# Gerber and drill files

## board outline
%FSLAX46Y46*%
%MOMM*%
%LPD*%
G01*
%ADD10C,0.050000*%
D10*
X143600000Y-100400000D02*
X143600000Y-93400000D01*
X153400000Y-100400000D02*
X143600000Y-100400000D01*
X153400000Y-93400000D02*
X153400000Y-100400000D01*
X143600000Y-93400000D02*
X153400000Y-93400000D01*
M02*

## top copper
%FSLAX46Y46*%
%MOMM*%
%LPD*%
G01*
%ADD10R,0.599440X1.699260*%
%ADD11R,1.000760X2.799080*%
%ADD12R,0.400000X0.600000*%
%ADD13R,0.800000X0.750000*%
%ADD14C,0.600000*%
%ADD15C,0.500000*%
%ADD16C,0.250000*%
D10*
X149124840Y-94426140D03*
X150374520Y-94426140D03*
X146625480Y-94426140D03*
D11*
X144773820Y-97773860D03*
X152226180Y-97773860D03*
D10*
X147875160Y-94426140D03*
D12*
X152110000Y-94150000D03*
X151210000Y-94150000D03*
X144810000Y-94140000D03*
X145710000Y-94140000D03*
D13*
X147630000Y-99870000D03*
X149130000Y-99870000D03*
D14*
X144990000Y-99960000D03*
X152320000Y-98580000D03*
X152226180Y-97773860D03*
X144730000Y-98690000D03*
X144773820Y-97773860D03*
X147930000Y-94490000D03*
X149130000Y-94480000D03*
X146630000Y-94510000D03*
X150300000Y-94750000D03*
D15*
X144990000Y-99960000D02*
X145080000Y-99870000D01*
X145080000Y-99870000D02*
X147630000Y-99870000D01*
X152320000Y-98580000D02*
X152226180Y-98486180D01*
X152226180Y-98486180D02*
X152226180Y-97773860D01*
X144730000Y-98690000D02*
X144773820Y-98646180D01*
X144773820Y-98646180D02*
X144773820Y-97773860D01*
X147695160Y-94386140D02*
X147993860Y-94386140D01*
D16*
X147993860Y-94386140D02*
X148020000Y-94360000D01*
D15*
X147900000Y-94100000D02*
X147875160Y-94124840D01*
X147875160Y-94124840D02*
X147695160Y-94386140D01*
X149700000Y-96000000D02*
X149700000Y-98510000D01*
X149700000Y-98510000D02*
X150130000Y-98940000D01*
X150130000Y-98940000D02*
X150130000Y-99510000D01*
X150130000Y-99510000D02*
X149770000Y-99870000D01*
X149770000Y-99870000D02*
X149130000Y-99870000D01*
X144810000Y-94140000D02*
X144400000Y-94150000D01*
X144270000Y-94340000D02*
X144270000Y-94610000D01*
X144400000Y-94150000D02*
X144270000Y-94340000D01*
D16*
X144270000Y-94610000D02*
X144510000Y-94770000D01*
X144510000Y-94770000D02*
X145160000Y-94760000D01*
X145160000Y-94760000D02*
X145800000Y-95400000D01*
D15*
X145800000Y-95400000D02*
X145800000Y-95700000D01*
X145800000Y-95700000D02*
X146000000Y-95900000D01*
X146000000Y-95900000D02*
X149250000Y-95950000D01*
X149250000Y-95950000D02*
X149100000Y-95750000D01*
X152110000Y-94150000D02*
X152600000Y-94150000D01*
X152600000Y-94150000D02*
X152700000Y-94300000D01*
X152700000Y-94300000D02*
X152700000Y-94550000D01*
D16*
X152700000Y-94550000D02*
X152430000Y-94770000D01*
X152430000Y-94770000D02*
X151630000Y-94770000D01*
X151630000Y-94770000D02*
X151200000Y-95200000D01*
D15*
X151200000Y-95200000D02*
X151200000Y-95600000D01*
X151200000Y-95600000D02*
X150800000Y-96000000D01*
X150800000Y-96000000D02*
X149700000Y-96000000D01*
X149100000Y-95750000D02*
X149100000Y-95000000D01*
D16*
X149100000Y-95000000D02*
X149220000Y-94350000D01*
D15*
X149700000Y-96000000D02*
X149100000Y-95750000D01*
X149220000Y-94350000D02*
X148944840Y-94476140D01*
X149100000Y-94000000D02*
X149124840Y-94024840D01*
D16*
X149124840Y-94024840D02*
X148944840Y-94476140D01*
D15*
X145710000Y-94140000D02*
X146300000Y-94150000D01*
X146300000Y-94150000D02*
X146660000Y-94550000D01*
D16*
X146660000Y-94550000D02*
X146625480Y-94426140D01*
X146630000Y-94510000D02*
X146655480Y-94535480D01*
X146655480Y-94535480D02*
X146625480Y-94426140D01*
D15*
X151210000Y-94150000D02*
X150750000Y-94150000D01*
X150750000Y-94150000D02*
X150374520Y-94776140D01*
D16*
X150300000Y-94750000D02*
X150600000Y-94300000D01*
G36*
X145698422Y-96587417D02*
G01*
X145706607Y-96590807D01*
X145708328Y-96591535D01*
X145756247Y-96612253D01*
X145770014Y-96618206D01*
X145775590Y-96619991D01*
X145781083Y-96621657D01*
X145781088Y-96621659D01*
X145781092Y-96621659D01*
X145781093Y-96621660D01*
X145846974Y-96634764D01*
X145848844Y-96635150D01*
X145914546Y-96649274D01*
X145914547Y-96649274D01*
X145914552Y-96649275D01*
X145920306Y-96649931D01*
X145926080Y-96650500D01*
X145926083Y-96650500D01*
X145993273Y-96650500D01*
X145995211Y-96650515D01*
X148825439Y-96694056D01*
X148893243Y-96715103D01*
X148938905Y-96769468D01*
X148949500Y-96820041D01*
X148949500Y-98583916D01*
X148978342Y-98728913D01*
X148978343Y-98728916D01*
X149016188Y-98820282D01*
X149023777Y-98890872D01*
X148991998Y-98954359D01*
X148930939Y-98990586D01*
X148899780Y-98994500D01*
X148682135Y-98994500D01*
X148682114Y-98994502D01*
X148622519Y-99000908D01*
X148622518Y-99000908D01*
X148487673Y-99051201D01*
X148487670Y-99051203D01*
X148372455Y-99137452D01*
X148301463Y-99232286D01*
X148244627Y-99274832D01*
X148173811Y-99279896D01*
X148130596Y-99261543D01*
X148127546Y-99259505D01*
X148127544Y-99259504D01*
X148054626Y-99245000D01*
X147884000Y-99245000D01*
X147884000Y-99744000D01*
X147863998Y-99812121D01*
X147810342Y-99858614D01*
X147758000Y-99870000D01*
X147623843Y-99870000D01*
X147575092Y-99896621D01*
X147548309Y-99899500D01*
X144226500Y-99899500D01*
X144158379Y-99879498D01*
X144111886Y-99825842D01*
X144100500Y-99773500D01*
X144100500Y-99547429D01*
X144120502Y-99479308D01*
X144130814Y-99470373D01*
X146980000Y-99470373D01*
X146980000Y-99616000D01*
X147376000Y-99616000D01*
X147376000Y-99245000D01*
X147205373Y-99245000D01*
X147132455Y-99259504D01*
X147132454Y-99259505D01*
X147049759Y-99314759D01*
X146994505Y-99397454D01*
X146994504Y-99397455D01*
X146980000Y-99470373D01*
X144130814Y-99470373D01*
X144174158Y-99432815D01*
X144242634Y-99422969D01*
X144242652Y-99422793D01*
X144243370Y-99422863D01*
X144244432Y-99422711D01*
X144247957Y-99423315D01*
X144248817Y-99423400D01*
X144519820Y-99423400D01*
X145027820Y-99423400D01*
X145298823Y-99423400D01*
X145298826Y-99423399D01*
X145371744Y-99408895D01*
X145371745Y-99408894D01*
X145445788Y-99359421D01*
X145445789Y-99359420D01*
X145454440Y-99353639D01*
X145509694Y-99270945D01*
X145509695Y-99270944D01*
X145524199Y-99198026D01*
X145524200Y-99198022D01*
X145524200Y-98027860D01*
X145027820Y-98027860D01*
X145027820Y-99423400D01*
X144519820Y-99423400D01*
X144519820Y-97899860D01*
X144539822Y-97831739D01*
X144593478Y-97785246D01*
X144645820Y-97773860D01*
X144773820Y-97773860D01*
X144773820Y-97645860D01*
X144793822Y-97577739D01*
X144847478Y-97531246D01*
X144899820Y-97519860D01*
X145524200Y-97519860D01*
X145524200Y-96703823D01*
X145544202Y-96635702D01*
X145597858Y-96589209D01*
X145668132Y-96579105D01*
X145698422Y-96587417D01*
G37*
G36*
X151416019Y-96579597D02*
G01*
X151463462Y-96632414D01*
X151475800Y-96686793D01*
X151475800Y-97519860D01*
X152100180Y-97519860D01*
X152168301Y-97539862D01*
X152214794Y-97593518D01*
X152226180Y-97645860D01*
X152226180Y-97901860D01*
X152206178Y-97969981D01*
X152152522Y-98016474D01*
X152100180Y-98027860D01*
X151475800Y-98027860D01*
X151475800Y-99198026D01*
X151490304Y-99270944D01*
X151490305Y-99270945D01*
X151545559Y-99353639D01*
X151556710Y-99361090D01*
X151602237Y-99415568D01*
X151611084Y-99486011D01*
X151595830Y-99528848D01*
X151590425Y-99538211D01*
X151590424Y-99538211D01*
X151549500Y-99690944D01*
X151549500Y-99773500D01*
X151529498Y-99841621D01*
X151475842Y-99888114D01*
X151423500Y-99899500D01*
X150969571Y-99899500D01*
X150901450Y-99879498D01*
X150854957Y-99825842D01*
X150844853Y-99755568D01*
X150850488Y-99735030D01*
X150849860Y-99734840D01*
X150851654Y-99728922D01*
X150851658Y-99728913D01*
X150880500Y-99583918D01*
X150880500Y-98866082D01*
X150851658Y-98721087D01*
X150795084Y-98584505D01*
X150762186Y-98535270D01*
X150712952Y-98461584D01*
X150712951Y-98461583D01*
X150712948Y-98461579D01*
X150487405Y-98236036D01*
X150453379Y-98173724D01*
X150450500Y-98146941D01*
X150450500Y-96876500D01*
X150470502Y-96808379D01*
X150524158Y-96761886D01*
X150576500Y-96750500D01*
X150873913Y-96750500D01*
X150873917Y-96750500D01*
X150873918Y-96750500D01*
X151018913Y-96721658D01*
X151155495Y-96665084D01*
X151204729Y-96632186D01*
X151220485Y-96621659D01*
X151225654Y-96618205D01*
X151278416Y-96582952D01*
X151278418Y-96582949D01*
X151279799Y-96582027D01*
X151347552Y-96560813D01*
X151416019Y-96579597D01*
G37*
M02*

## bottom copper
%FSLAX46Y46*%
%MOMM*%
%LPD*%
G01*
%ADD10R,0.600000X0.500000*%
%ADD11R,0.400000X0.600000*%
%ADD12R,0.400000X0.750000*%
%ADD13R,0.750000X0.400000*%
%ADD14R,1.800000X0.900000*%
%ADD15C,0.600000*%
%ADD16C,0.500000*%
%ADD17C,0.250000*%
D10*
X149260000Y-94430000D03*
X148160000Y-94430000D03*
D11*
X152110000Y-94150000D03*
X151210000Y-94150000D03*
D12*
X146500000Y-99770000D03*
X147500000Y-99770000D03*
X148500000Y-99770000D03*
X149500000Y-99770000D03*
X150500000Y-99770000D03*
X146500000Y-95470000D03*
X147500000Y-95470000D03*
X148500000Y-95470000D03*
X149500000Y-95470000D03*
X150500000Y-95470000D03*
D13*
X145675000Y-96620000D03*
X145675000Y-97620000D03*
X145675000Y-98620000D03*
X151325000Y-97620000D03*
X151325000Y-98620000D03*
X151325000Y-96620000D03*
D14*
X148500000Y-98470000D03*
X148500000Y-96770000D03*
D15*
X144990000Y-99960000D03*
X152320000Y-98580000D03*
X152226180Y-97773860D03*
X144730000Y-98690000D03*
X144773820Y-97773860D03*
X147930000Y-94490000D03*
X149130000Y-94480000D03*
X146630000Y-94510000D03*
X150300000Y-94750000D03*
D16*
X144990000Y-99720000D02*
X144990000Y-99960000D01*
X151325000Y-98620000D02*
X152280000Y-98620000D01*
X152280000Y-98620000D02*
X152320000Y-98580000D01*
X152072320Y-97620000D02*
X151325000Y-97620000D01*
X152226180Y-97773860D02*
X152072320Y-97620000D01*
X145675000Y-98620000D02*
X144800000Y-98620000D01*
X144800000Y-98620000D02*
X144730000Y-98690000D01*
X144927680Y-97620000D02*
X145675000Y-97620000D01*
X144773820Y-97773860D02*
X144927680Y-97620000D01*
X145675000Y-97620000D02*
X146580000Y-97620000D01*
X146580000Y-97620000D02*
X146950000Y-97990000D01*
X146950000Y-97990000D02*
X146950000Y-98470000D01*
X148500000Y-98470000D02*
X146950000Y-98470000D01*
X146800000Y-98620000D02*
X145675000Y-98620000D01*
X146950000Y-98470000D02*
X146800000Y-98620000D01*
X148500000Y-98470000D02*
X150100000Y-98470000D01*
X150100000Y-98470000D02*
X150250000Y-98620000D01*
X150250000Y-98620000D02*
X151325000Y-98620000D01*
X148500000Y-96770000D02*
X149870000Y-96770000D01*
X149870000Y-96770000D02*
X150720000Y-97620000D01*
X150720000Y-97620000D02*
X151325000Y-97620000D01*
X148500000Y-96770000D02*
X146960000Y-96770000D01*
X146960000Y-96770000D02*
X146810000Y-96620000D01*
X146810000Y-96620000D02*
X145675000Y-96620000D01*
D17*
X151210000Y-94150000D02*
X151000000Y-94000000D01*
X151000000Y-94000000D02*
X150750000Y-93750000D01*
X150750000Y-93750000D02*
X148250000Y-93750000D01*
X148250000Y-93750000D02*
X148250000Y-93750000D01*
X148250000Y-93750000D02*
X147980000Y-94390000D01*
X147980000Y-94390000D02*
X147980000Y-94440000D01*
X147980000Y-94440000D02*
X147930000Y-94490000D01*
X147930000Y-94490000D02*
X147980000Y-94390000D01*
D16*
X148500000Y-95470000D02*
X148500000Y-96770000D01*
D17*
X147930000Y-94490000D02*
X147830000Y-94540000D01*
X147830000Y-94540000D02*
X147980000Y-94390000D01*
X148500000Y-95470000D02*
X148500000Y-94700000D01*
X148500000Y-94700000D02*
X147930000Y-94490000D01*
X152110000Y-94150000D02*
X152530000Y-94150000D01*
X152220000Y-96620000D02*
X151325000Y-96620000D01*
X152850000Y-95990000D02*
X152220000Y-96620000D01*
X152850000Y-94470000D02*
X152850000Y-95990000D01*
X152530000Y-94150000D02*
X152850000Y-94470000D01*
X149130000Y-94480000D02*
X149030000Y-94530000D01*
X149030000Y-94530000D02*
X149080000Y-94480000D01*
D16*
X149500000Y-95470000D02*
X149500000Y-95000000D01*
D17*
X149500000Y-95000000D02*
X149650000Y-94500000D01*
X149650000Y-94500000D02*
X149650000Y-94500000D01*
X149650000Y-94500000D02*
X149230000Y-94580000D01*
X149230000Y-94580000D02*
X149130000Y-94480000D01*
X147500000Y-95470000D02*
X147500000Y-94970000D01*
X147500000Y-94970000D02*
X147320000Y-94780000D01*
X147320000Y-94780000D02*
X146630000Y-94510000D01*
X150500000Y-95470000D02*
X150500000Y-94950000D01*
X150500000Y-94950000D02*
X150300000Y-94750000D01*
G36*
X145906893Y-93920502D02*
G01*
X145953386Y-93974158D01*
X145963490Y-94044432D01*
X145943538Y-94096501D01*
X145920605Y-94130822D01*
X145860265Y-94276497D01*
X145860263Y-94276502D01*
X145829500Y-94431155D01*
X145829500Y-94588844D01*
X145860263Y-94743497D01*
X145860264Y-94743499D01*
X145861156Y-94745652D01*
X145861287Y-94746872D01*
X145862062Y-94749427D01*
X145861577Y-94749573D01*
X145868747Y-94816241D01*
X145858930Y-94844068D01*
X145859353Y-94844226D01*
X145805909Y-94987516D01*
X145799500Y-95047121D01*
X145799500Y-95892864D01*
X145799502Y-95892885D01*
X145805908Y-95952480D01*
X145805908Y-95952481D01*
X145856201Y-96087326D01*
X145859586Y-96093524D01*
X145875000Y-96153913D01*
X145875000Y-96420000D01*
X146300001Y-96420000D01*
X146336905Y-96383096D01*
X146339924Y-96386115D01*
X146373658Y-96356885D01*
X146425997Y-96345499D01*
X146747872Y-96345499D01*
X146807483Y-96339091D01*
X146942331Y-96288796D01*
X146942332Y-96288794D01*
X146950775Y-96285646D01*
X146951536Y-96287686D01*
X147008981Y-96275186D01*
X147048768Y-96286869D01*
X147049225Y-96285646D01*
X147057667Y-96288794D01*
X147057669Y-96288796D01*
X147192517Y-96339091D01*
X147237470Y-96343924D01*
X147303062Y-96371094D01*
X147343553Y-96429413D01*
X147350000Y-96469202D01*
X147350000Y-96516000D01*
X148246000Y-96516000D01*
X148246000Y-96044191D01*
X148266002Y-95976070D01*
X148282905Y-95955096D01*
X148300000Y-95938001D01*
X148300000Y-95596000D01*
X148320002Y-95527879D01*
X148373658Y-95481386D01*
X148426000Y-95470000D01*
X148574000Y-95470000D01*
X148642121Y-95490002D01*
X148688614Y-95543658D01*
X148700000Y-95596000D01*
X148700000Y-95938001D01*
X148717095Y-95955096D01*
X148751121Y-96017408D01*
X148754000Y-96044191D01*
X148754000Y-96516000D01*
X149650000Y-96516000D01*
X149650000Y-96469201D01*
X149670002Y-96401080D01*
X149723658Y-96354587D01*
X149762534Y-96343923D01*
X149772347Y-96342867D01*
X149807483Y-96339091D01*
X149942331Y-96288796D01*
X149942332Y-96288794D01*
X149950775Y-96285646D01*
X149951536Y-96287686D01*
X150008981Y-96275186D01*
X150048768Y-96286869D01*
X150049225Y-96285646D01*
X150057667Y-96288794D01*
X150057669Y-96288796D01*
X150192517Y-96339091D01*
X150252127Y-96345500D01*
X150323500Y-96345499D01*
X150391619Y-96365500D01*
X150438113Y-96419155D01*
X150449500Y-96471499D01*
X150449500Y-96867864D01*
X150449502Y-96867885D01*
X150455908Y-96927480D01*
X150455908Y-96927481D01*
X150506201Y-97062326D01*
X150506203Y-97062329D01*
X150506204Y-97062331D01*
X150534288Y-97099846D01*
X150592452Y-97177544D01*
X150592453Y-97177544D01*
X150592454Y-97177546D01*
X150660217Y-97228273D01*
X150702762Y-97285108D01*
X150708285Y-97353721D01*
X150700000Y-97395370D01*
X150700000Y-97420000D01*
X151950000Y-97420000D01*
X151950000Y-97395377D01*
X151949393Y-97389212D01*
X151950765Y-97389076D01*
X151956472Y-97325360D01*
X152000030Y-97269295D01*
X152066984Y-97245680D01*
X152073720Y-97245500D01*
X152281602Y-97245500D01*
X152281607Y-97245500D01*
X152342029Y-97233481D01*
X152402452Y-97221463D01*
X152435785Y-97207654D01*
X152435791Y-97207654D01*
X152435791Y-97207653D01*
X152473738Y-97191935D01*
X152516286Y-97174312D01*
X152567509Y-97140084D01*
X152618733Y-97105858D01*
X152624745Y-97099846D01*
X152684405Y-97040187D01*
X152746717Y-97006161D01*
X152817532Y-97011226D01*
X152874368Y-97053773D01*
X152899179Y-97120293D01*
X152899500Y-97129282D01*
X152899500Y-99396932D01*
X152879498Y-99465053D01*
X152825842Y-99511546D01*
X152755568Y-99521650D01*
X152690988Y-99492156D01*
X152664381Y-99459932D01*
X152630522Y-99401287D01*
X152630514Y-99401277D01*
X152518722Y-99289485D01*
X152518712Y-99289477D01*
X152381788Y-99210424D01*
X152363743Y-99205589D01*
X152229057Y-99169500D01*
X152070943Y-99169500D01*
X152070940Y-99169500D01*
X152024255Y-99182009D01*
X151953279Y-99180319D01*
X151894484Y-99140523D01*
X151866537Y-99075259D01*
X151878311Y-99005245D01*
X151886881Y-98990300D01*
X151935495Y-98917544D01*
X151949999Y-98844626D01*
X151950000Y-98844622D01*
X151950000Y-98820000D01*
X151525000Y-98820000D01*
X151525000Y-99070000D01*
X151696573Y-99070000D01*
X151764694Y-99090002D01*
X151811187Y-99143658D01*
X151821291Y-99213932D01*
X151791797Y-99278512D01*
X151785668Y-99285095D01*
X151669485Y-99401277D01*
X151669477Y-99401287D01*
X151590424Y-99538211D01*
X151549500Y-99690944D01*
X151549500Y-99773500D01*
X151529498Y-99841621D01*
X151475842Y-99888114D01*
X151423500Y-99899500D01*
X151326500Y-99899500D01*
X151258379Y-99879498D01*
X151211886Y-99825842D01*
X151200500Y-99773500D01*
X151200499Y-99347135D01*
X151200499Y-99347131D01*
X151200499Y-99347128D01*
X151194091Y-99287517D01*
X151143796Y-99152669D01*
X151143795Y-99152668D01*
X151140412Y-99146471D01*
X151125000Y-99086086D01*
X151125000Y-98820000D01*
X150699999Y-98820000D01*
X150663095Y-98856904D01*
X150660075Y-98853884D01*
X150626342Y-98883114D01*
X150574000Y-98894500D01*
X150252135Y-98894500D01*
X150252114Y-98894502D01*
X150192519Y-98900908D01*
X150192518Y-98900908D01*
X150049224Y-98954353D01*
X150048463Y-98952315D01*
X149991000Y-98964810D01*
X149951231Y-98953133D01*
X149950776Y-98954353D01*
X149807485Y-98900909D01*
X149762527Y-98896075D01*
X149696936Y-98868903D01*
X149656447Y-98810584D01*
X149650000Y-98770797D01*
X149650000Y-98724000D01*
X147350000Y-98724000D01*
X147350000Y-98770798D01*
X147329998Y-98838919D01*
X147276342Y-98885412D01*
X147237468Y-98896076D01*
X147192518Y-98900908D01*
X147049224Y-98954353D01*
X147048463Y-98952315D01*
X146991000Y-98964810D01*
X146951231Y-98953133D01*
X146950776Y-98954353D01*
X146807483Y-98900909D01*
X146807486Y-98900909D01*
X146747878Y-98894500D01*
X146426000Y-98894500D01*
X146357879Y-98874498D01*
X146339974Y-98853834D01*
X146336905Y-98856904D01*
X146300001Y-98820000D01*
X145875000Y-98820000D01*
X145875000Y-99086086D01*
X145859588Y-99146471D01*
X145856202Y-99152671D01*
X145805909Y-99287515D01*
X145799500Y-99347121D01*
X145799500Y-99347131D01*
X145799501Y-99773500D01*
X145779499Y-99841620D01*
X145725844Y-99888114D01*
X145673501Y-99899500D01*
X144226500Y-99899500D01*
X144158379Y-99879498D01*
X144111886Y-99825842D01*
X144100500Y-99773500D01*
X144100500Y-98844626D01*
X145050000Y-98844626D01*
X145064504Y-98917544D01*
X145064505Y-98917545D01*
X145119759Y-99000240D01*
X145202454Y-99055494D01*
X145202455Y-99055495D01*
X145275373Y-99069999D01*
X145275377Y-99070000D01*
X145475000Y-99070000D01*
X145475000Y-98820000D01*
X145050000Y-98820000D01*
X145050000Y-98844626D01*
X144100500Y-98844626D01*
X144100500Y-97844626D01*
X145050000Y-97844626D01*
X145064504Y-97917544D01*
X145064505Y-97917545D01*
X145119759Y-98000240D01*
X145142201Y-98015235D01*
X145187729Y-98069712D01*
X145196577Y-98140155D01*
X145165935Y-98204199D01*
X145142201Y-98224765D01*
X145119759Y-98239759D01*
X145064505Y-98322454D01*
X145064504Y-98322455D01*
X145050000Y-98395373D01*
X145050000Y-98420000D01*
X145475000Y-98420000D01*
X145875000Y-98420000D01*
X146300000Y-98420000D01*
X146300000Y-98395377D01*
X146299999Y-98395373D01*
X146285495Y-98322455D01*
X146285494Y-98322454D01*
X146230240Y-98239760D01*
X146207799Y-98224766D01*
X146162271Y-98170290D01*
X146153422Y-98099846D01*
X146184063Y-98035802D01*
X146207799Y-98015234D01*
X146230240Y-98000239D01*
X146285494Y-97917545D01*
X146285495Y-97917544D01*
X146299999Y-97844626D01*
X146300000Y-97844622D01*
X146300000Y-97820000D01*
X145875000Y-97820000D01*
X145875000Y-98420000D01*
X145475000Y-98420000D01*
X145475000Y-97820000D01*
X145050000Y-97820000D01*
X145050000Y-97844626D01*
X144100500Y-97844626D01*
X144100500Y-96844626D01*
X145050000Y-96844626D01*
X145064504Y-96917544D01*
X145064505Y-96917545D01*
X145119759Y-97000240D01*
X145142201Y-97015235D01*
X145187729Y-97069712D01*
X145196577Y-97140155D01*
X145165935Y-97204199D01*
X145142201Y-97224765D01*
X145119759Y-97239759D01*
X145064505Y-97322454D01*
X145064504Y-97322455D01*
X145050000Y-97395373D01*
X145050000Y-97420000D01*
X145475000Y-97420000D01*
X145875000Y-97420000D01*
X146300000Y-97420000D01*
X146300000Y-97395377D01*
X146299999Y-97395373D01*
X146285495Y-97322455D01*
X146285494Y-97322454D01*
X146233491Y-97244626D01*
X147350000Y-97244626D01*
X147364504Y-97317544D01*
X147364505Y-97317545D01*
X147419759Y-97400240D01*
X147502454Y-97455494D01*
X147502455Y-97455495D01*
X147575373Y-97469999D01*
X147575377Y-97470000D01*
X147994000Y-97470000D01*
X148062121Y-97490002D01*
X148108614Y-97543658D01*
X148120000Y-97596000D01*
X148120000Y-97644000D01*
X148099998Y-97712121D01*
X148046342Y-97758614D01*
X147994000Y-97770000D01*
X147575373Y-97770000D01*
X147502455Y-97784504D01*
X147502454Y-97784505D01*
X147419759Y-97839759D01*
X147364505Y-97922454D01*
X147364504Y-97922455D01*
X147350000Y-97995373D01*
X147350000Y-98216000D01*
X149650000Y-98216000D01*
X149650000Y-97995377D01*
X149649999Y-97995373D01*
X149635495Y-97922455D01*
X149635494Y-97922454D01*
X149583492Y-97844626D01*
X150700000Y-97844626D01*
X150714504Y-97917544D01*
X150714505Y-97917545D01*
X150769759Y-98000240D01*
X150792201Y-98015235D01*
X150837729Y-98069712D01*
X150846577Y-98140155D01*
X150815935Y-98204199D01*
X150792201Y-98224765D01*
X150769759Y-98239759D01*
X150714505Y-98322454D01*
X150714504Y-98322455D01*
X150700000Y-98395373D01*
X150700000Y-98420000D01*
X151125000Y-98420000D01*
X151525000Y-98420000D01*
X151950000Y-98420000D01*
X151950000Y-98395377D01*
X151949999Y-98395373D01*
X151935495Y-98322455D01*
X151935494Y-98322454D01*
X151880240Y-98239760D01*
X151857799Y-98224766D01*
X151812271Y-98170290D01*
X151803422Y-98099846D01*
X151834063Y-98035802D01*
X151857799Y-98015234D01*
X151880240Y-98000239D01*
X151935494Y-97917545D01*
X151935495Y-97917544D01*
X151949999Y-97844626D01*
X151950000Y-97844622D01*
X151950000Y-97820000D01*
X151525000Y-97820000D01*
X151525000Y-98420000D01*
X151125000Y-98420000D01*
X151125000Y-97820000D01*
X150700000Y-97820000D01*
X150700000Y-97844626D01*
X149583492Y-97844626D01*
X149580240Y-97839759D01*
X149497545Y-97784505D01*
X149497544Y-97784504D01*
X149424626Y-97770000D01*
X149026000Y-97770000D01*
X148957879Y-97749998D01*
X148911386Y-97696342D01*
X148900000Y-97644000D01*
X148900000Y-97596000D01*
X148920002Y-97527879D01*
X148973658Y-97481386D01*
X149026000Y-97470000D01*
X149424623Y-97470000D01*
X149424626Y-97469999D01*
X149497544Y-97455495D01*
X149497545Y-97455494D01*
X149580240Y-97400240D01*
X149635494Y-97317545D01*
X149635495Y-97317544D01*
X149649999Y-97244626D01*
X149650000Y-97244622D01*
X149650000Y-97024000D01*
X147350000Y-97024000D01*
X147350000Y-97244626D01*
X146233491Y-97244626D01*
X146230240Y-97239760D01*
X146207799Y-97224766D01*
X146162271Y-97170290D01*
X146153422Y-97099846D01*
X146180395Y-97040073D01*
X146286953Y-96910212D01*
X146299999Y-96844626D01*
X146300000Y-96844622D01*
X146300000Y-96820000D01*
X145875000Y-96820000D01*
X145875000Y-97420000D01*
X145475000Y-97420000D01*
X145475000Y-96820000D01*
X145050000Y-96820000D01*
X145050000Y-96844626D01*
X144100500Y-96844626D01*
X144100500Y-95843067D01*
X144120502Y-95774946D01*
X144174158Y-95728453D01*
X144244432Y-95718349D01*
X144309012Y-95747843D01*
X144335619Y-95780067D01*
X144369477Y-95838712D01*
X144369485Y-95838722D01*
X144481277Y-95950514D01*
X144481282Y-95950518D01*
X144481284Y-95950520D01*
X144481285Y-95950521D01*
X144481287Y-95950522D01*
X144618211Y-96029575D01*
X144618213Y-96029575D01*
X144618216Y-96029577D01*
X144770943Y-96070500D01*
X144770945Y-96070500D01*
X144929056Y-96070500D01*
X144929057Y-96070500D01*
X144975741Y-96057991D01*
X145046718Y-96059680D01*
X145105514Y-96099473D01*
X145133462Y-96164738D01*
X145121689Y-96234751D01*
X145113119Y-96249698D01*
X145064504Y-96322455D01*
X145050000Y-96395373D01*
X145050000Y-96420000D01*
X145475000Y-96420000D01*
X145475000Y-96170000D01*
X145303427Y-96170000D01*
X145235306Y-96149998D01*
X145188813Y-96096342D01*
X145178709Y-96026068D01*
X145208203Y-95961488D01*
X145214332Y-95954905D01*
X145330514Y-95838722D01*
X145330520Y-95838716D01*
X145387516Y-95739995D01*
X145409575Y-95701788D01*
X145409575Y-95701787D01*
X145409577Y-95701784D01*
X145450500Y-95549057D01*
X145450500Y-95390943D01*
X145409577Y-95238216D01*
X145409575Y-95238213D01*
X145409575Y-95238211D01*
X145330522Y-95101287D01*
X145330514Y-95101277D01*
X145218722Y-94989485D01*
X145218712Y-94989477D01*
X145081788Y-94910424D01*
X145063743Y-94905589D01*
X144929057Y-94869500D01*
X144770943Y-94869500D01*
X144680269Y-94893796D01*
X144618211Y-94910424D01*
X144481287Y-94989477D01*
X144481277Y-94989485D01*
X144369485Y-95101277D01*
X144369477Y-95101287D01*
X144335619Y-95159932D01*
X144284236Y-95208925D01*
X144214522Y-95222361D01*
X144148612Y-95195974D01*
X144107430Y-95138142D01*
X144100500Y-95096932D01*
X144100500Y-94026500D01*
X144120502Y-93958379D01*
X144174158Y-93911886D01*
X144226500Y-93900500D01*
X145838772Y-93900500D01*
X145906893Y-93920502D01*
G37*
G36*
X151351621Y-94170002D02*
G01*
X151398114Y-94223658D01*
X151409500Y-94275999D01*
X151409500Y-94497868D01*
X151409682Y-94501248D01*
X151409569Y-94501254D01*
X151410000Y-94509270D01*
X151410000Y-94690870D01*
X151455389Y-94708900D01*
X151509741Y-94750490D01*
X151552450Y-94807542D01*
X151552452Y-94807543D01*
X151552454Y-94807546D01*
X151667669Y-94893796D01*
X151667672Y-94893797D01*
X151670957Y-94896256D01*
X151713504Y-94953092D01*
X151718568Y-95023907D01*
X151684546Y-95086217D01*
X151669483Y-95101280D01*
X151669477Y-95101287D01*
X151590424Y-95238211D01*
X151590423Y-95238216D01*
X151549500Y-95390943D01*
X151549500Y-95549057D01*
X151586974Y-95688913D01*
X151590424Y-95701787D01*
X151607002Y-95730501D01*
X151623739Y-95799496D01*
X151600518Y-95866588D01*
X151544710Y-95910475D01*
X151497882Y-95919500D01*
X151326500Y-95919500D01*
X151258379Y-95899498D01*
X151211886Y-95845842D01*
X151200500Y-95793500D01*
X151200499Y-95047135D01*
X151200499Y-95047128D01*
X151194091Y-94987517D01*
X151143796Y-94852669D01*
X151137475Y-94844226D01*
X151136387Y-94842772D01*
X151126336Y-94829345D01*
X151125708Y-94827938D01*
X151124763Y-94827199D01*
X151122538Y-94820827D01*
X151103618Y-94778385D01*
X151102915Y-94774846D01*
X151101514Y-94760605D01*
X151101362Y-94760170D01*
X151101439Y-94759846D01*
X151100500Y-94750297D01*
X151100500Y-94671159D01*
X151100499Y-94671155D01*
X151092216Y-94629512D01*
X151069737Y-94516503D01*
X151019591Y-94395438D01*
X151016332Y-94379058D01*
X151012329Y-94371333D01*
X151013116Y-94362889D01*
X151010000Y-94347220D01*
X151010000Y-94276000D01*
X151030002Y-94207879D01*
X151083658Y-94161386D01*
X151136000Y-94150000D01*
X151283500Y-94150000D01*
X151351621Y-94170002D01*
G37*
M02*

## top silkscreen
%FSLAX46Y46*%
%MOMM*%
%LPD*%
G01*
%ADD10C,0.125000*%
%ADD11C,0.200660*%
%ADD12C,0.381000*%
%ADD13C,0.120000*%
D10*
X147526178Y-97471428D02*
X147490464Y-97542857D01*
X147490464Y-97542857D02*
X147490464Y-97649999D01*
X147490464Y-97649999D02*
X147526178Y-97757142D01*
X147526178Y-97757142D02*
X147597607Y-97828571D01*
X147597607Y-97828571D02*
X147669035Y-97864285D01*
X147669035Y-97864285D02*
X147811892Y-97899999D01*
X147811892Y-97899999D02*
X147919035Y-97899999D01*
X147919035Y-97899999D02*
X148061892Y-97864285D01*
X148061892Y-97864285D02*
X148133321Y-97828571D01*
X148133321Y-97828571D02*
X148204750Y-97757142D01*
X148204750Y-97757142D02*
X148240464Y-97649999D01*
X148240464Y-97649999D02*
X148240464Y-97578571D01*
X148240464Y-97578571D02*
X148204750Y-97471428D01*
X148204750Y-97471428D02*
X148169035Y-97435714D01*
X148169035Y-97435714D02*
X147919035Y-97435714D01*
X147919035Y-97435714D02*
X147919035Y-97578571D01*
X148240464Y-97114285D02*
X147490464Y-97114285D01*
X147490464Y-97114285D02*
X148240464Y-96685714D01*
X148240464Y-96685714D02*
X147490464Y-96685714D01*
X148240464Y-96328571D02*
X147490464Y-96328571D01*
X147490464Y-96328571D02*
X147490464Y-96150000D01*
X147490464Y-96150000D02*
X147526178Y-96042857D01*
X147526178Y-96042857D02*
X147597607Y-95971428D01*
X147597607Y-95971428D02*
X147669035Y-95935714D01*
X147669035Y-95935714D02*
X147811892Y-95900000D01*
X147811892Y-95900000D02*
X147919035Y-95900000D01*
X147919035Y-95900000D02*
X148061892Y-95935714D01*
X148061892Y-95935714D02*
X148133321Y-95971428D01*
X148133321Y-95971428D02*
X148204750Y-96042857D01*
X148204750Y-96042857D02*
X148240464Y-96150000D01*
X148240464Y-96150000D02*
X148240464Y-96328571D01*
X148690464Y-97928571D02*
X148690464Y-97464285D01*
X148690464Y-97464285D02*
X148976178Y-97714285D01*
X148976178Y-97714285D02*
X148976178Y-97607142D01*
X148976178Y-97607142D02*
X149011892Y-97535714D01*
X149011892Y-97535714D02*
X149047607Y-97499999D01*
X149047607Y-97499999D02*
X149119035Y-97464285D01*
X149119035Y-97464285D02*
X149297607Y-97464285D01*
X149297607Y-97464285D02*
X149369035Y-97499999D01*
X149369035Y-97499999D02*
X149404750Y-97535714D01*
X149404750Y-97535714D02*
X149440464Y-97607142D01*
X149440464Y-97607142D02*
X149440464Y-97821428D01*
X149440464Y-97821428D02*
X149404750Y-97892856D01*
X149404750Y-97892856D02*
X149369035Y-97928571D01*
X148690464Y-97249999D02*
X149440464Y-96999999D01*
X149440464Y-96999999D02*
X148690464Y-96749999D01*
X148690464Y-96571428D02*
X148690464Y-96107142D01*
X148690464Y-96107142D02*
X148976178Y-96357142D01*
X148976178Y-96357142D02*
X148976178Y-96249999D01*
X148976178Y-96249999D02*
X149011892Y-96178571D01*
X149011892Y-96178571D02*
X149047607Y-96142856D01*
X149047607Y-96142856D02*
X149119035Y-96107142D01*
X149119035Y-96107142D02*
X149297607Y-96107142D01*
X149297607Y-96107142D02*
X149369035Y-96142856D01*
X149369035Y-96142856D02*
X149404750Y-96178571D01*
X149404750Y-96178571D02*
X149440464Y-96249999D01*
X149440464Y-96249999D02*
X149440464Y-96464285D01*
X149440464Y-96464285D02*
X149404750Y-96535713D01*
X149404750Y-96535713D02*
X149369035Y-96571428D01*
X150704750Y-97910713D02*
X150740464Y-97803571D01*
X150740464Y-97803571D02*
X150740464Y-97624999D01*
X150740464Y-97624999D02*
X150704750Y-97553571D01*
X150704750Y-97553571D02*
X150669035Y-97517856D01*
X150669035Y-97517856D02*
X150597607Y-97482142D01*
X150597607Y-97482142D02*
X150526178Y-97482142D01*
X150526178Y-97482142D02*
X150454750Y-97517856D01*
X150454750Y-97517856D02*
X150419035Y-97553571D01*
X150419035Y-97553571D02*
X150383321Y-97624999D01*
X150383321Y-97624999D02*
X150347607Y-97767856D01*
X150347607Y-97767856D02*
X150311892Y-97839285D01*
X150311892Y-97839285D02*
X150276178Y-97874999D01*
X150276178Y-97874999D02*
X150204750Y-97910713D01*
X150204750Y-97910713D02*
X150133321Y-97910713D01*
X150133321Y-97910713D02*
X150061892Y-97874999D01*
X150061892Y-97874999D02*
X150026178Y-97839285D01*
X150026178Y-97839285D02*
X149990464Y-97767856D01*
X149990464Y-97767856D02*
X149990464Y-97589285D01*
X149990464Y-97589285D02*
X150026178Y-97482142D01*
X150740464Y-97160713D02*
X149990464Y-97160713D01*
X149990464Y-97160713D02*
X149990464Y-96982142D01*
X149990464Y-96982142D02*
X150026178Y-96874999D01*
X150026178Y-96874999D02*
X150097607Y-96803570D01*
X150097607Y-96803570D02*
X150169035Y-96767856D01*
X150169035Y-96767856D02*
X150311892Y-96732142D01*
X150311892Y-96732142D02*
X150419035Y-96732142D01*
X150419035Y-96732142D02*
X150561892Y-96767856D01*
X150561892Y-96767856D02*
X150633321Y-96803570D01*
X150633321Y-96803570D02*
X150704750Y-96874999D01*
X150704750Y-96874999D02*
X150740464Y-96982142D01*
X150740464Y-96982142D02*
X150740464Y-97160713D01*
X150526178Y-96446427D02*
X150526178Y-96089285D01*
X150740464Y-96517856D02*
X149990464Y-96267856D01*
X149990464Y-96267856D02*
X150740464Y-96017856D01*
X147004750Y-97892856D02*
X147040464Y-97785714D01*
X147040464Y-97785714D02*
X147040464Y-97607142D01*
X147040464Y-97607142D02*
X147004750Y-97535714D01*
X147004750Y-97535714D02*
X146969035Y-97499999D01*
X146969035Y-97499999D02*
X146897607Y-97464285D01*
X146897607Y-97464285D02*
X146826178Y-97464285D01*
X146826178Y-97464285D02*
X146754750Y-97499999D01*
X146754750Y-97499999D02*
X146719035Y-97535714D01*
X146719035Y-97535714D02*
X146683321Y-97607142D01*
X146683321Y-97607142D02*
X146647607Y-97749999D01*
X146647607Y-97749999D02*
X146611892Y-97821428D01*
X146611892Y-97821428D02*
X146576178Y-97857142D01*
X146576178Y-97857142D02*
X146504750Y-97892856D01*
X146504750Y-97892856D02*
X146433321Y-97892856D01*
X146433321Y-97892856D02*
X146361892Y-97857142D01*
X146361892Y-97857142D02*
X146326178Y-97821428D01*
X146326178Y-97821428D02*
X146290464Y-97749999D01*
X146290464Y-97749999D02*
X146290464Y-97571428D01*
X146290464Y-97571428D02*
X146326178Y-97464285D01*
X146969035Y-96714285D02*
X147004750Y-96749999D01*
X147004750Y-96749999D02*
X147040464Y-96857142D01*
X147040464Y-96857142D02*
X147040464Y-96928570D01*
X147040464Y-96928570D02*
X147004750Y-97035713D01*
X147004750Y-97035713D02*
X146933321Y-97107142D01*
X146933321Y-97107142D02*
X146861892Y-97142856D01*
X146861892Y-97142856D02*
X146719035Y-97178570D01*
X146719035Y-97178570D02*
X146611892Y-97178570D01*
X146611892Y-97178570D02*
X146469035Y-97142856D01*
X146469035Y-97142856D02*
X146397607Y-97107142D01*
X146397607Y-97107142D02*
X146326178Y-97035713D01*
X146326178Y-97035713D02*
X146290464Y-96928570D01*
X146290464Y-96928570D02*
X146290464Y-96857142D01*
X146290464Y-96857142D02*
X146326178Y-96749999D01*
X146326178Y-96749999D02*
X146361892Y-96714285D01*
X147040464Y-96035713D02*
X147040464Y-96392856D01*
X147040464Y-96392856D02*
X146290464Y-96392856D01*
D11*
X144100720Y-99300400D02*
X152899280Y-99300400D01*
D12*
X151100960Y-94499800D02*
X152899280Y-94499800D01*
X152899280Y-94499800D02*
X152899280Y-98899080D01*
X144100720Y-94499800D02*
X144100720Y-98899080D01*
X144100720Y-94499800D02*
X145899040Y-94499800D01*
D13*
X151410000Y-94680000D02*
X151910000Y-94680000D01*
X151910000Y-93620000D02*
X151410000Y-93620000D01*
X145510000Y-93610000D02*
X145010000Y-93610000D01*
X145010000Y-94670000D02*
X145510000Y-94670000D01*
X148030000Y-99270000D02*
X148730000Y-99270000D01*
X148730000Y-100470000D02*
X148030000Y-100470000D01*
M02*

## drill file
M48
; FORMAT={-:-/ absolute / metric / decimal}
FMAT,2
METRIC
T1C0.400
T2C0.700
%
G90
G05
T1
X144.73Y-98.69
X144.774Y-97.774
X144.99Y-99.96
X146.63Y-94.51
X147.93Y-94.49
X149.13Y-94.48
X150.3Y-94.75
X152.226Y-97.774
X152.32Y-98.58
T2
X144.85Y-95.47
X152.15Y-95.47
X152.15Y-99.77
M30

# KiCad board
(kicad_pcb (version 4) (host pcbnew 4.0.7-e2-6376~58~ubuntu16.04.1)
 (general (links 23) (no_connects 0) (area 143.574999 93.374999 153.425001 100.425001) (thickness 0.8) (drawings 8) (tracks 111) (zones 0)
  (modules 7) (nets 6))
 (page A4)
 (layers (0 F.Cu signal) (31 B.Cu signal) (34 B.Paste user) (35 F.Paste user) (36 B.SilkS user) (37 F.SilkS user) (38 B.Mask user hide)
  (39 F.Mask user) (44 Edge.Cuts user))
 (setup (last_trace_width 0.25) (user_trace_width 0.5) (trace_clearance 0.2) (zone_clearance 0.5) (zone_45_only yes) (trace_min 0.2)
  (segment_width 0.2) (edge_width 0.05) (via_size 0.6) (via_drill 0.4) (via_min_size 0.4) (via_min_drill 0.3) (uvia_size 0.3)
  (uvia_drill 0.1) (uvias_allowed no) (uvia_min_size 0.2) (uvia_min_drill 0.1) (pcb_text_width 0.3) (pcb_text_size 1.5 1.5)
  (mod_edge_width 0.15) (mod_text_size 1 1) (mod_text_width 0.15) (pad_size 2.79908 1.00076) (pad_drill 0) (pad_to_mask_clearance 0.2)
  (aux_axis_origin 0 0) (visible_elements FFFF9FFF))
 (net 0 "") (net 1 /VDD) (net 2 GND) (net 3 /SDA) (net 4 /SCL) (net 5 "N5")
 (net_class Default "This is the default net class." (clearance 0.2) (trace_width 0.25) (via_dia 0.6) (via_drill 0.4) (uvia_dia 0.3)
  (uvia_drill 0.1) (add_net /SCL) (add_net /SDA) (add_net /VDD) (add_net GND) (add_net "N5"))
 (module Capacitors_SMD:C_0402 (layer B.Cu) (at 148.71 94.43 180)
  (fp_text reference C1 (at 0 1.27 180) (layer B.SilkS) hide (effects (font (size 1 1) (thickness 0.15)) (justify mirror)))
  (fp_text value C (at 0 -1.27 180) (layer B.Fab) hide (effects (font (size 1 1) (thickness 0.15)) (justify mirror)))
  (pad 1 smd rect (at -0.55 0 180) (size 0.6 0.5) (layers B.Cu B.Paste B.Mask) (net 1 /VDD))
  (pad 2 smd rect (at 0.55 0 180) (size 0.6 0.5) (layers B.Cu B.Paste B.Mask) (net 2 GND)))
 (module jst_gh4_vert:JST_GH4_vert (layer F.Cu) (at 148.5 96.1 90)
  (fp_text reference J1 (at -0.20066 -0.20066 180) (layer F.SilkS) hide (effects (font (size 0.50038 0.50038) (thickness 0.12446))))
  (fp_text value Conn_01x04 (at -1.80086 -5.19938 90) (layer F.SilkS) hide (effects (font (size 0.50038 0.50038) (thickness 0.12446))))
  (fp_line (start -3.2004 -4.39928) (end -3.2004 4.39928) (layer F.SilkS) (width 0.20066))
  (fp_line (start 1.6002 2.60096) (end 1.6002 4.39928) (layer F.SilkS) (width 0.381))
  (fp_line (start 1.6002 4.39928) (end -2.79908 4.39928) (layer F.SilkS) (width 0.381))
  (fp_line (start 1.6002 -4.39928) (end -2.79908 -4.39928) (layer F.SilkS) (width 0.381))
  (fp_line (start 1.6002 -4.39928) (end 1.6002 -2.60096) (layer F.SilkS) (width 0.381))
  (pad 3 smd rect (at 1.67386 0.62484) (size 0.59944 1.69926) (layers F.Cu F.Paste F.Mask) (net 1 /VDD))
  (pad 4 smd rect (at 1.67386 1.87452) (size 0.59944 1.69926) (layers F.Cu F.Paste F.Mask) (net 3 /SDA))
  (pad 1 smd rect (at 1.67386 -1.87452) (size 0.59944 1.69926) (layers F.Cu F.Paste F.Mask) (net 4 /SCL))
  (pad "" smd rect (at -1.67386 -3.72618 90) (size 2.79908 1.00076) (layers F.Cu F.Paste F.Mask) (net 2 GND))
  (pad "" smd rect (at -1.67386 3.72618 90) (size 2.79908 1.00076) (layers F.Cu F.Paste F.Mask) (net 2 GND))
  (pad 2 smd rect (at 1.67386 -0.62484) (size 0.59944 1.69926) (layers F.Cu F.Paste F.Mask) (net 2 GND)))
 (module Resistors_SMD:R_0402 (layer F.Cu) (at 151.66 94.15 180)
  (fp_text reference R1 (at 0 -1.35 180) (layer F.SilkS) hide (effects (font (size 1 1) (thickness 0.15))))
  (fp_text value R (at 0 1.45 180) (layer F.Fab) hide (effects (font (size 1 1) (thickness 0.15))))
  (fp_line (start 0.25 -0.53) (end -0.25 -0.53) (layer F.SilkS) (width 0.12))
  (fp_line (start -0.25 0.53) (end 0.25 0.53) (layer F.SilkS) (width 0.12))
  (pad 1 smd rect (at -0.45 0 180) (size 0.4 0.6) (layers F.Cu F.Paste F.Mask) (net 1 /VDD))
  (pad 2 smd rect (at 0.45 0 180) (size 0.4 0.6) (layers F.Cu F.Paste F.Mask) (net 3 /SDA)))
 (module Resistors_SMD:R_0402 (layer F.Cu) (at 145.26 94.14)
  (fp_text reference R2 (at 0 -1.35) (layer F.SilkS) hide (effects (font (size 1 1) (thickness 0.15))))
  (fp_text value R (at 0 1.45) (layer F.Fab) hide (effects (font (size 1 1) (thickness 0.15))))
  (fp_line (start 0.25 -0.53) (end -0.25 -0.53) (layer F.SilkS) (width 0.12))
  (fp_line (start -0.25 0.53) (end 0.25 0.53) (layer F.SilkS) (width 0.12))
  (pad 1 smd rect (at -0.45 0) (size 0.4 0.6) (layers F.Cu F.Paste F.Mask) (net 1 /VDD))
  (pad 2 smd rect (at 0.45 0) (size 0.4 0.6) (layers F.Cu F.Paste F.Mask) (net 4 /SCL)))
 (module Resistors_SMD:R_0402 (layer B.Cu) (at 151.66 94.15 180)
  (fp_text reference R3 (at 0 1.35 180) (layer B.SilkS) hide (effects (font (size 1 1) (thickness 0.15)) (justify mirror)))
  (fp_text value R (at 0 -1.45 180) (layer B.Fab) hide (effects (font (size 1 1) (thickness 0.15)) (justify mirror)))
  (pad 1 smd rect (at -0.45 0 180) (size 0.4 0.6) (layers B.Cu B.Paste B.Mask) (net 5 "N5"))
  (pad 2 smd rect (at 0.45 0 180) (size 0.4 0.6) (layers B.Cu B.Paste B.Mask) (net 2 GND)))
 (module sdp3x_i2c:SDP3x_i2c (layer B.Cu) (at 148.5 97.62)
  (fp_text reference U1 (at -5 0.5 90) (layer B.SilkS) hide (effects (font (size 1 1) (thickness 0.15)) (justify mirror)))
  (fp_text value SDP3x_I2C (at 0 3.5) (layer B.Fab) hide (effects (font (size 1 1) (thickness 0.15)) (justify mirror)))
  (pad 16 smd rect (at -2 2.15) (size 0.4 0.75) (layers B.Cu B.Paste B.Mask))
  (pad 15 smd rect (at -1 2.15) (size 0.4 0.75) (layers B.Cu B.Paste B.Mask))
  (pad 14 smd rect (at 0 2.15) (size 0.4 0.75) (layers B.Cu B.Paste B.Mask))
  (pad 13 smd rect (at 1 2.15) (size 0.4 0.75) (layers B.Cu B.Paste B.Mask))
  (pad 12 smd rect (at 2 2.15) (size 0.4 0.75) (layers B.Cu B.Paste B.Mask))
  (pad 4 smd rect (at -2 -2.15) (size 0.4 0.75) (layers B.Cu B.Paste B.Mask))
  (pad 5 smd rect (at -1 -2.15) (size 0.4 0.75) (layers B.Cu B.Paste B.Mask) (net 4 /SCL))
  (pad 6 smd rect (at 0 -2.15) (size 0.4 0.75) (layers B.Cu B.Paste B.Mask) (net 2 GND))
  (pad 7 smd rect (at 1 -2.15) (size 0.4 0.75) (layers B.Cu B.Paste B.Mask) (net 1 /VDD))
  (pad 8 smd rect (at 2 -2.15) (size 0.4 0.75) (layers B.Cu B.Paste B.Mask) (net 3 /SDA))
  (pad 3 smd rect (at -2.825 -1) (size 0.75 0.4) (layers B.Cu B.Paste B.Mask) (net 2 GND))
  (pad 2 smd rect (at -2.825 0) (size 0.75 0.4) (layers B.Cu B.Paste B.Mask) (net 2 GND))
  (pad 1 smd rect (at -2.825 1) (size 0.75 0.4) (layers B.Cu B.Paste B.Mask) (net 2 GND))
  (pad 10 smd rect (at 2.825 0) (size 0.75 0.4) (layers B.Cu B.Paste B.Mask) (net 2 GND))
  (pad 11 smd rect (at 2.825 1) (size 0.75 0.4) (layers B.Cu B.Paste B.Mask) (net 2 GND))
  (pad 9 smd rect (at 2.825 -1) (size 0.75 0.4) (layers B.Cu B.Paste B.Mask) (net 5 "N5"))
  (pad 1 smd rect (at 0 0.85) (size 1.8 0.9) (layers B.Cu B.Paste B.Mask) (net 2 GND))
  (pad 1 smd rect (at 0 -0.85) (size 1.8 0.9) (layers B.Cu B.Paste B.Mask) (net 2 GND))
  (pad "" np_thru_hole circle (at 3.65 -2.15) (size 0.7 0.7) (drill 0.7) (layers *.Cu *.Mask) (zone_connect 0))
  (pad "" np_thru_hole circle (at 3.65 2.15) (size 0.7 0.7) (drill 0.7) (layers *.Cu *.Mask))
  (pad "" np_thru_hole circle (at -3.65 -2.15) (size 0.7 0.7) (drill 0.7) (layers *.Cu *.Mask)))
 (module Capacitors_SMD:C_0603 (layer F.Cu) (at 148.38 99.87 180)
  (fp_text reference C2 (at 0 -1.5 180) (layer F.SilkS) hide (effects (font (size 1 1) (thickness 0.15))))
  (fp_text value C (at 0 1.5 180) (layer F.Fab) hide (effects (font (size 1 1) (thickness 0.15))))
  (fp_line (start 0.35 0.6) (end -0.35 0.6) (layer F.SilkS) (width 0.12))
  (fp_line (start -0.35 -0.6) (end 0.35 -0.6) (layer F.SilkS) (width 0.12))
  (pad 2 smd rect (at 0.75 0 180) (size 0.8 0.75) (layers F.Cu F.Paste F.Mask) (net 2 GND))
  (pad 1 smd rect (at -0.75 0 180) (size 0.8 0.75) (layers F.Cu F.Paste F.Mask) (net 1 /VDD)))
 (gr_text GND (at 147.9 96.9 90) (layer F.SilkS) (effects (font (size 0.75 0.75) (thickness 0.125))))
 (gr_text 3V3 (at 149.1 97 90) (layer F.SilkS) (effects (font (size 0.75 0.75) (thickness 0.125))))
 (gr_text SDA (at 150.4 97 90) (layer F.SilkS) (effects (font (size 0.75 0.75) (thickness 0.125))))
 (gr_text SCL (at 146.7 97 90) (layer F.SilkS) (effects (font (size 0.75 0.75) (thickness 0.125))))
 (gr_line (start 143.6 100.4) (end 143.6 93.4) (angle 90) (layer Edge.Cuts) (width 0.05))
 (gr_line (start 153.4 100.4) (end 143.6 100.4) (angle 90) (layer Edge.Cuts) (width 0.05))
 (gr_line (start 153.4 93.4) (end 153.4 100.4) (angle 90) (layer Edge.Cuts) (width 0.05))
 (gr_line (start 143.6 93.4) (end 153.4 93.4) (angle 90) (layer Edge.Cuts) (width 0.05))
 (segment (start 144.99 99.72) (end 144.99 99.96) (width 0.5) (layer B.Cu) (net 2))
 (via (at 144.99 99.96) (size 0.6) (drill 0.4) (layers F.Cu B.Cu) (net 2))
 (segment (start 144.99 99.96) (end 145.08 99.87) (width 0.5) (layer F.Cu) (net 2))
 (segment (start 145.08 99.87) (end 147.63 99.87) (width 0.5) (layer F.Cu) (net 2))
 (segment (start 151.325 98.62) (end 152.28 98.62) (width 0.5) (layer B.Cu) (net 2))
 (segment (start 152.28 98.62) (end 152.32 98.58) (width 0.5) (layer B.Cu) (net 2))
 (via (at 152.32 98.58) (size 0.6) (drill 0.4) (layers F.Cu B.Cu) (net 2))
 (segment (start 152.32 98.58) (end 152.22618 98.48618) (width 0.5) (layer F.Cu) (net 2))
 (segment (start 152.22618 98.48618) (end 152.22618 97.77386) (width 0.5) (layer F.Cu) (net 2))
 (segment (start 152.07232 97.62) (end 151.325 97.62) (width 0.5) (layer B.Cu) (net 2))
 (segment (start 152.22618 97.77386) (end 152.07232 97.62) (width 0.5) (layer B.Cu) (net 2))
 (via (at 152.22618 97.77386) (size 0.6) (drill 0.4) (layers F.Cu B.Cu) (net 2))
 (segment (start 145.675 98.62) (end 144.8 98.62) (width 0.5) (layer B.Cu) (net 2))
 (segment (start 144.8 98.62) (end 144.73 98.69) (width 0.5) (layer B.Cu) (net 2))
 (via (at 144.73 98.69) (size 0.6) (drill 0.4) (layers F.Cu B.Cu) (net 2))
 (segment (start 144.73 98.69) (end 144.77382 98.64618) (width 0.5) (layer F.Cu) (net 2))
 (segment (start 144.77382 98.64618) (end 144.77382 97.77386) (width 0.5) (layer F.Cu) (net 2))
 (segment (start 144.92768 97.62) (end 145.675 97.62) (width 0.5) (layer B.Cu) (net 2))
 (segment (start 144.77382 97.77386) (end 144.92768 97.62) (width 0.5) (layer B.Cu) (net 2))
 (via (at 144.77382 97.77386) (size 0.6) (drill 0.4) (layers F.Cu B.Cu) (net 2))
 (segment (start 145.675 97.62) (end 146.58 97.62) (width 0.5) (layer B.Cu) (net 2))
 (segment (start 146.58 97.62) (end 146.95 97.99) (width 0.5) (layer B.Cu) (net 2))
 (segment (start 146.95 97.99) (end 146.95 98.47) (width 0.5) (layer B.Cu) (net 2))
 (segment (start 148.5 98.47) (end 146.95 98.47) (width 0.5) (layer B.Cu) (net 2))
 (segment (start 146.8 98.62) (end 145.675 98.62) (width 0.5) (layer B.Cu) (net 2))
 (segment (start 146.95 98.47) (end 146.8 98.62) (width 0.5) (layer B.Cu) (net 2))
 (segment (start 148.5 98.47) (end 150.1 98.47) (width 0.5) (layer B.Cu) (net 2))
 (segment (start 150.1 98.47) (end 150.25 98.62) (width 0.5) (layer B.Cu) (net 2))
 (segment (start 150.25 98.62) (end 151.325 98.62) (width 0.5) (layer B.Cu) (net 2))
 (segment (start 148.5 96.77) (end 149.87 96.77) (width 0.5) (layer B.Cu) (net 2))
 (segment (start 149.87 96.77) (end 150.72 97.62) (width 0.5) (layer B.Cu) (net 2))
 (segment (start 150.72 97.62) (end 151.325 97.62) (width 0.5) (layer B.Cu) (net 2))
 (segment (start 148.5 96.77) (end 146.96 96.77) (width 0.5) (layer B.Cu) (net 2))
 (segment (start 146.96 96.77) (end 146.81 96.62) (width 0.5) (layer B.Cu) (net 2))
 (segment (start 146.81 96.62) (end 145.675 96.62) (width 0.5) (layer B.Cu) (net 2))
 (segment (start 151.21 94.15) (end 151 94) (width 0.25) (layer B.Cu) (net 2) (status 10))
 (segment (start 151 94) (end 150.75 93.75) (width 0.25) (layer B.Cu) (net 2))
 (segment (start 150.75 93.75) (end 148.25 93.75) (width 0.25) (layer B.Cu) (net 2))
 (segment (start 148.25 93.75) (end 148.25 93.75) (width 0.25) (layer B.Cu) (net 2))
 (segment (start 148.25 93.75) (end 147.98 94.39) (width 0.25) (layer B.Cu) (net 2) (status 20))
 (segment (start 147.69516 94.38614) (end 147.99386 94.38614) (width 0.5) (layer F.Cu) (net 2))
 (segment (start 147.99386 94.38614) (end 148.02 94.36) (width 0.25) (layer F.Cu) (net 2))
 (via (at 147.93 94.49) (size 0.6) (drill 0.4) (layers F.Cu B.Cu) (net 2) (status 30))
 (segment (start 147.98 94.39) (end 147.98 94.44) (width 0.25) (layer B.Cu) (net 2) (status 30))
 (segment (start 147.98 94.44) (end 147.93 94.49) (width 0.25) (layer B.Cu) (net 2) (status 30))
 (segment (start 147.93 94.49) (end 147.98 94.39) (width 0.25) (layer B.Cu) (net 2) (status 30))
 (segment (start 148.5 95.47) (end 148.5 96.77) (width 0.5) (layer B.Cu) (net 2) (status 30))
 (segment (start 147.9 94.1) (end 147.87516 94.12484) (width 0.5) (layer F.Cu) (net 2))
 (segment (start 147.87516 94.12484) (end 147.69516 94.38614) (width 0.5) (layer F.Cu) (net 2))
 (segment (start 147.93 94.49) (end 147.83 94.54) (width 0.25) (layer B.Cu) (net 2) (status 30))
 (segment (start 147.83 94.54) (end 147.98 94.39) (width 0.25) (layer B.Cu) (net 2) (status 30))
 (segment (start 148.5 95.47) (end 148.5 94.7) (width 0.25) (layer B.Cu) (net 2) (status 10))
 (segment (start 148.5 94.7) (end 147.93 94.49) (width 0.25) (layer B.Cu) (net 2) (status 20))
 (segment (start 152.11 94.15) (end 152.53 94.15) (width 0.25) (layer B.Cu) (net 5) (status 10))
 (segment (start 152.22 96.62) (end 151.325 96.62) (width 0.25) (layer B.Cu) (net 5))
 (segment (start 152.85 95.99) (end 152.22 96.62) (width 0.25) (layer B.Cu) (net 5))
 (segment (start 152.85 94.47) (end 152.85 95.99) (width 0.25) (layer B.Cu) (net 5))
 (segment (start 152.53 94.15) (end 152.85 94.47) (width 0.25) (layer B.Cu) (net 5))
 (segment (start 149.7 96) (end 149.7 98.51) (width 0.5) (layer F.Cu) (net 1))
 (segment (start 149.7 98.51) (end 150.13 98.94) (width 0.5) (layer F.Cu) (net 1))
 (segment (start 150.13 98.94) (end 150.13 99.51) (width 0.5) (layer F.Cu) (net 1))
 (segment (start 150.13 99.51) (end 149.77 99.87) (width 0.5) (layer F.Cu) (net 1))
 (segment (start 149.77 99.87) (end 149.13 99.87) (width 0.5) (layer F.Cu) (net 1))
 (segment (start 144.81 94.14) (end 144.4 94.15) (width 0.5) (layer F.Cu) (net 1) (status 10))
 (segment (start 144.27 94.34) (end 144.27 94.61) (width 0.5) (layer F.Cu) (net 1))
 (segment (start 144.4 94.15) (end 144.27 94.34) (width 0.5) (layer F.Cu) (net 1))
 (segment (start 144.27 94.61) (end 144.51 94.77) (width 0.25) (layer F.Cu) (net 1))
 (segment (start 144.51 94.77) (end 145.16 94.76) (width 0.25) (layer F.Cu) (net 1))
 (segment (start 145.16 94.76) (end 145.8 95.4) (width 0.25) (layer F.Cu) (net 1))
 (segment (start 145.8 95.4) (end 145.8 95.7) (width 0.5) (layer F.Cu) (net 1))
 (segment (start 145.8 95.7) (end 146 95.9) (width 0.5) (layer F.Cu) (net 1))
 (segment (start 146 95.9) (end 149.25 95.95) (width 0.5) (layer F.Cu) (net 1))
 (segment (start 149.25 95.95) (end 149.1 95.75) (width 0.5) (layer F.Cu) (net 1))
 (segment (start 152.11 94.15) (end 152.6 94.15) (width 0.5) (layer F.Cu) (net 1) (status 10))
 (segment (start 152.6 94.15) (end 152.7 94.3) (width 0.5) (layer F.Cu) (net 1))
 (segment (start 152.7 94.3) (end 152.7 94.55) (width 0.5) (layer F.Cu) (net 1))
 (segment (start 152.7 94.55) (end 152.43 94.77) (width 0.25) (layer F.Cu) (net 1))
 (segment (start 152.43 94.77) (end 151.63 94.77) (width 0.25) (layer F.Cu) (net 1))
 (segment (start 151.63 94.77) (end 151.2 95.2) (width 0.25) (layer F.Cu) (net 1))
 (segment (start 151.2 95.2) (end 151.2 95.6) (width 0.5) (layer F.Cu) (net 1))
 (segment (start 151.2 95.6) (end 150.8 96) (width 0.5) (layer F.Cu) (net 1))
 (segment (start 150.8 96) (end 149.7 96) (width 0.5) (layer F.Cu) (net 1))
 (segment (start 149.1 95.75) (end 149.1 95) (width 0.5) (layer F.Cu) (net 1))
 (segment (start 149.1 95) (end 149.22 94.35) (width 0.25) (layer F.Cu) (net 1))
 (segment (start 149.7 96) (end 149.1 95.75) (width 0.5) (layer F.Cu) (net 1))
 (segment (start 149.22 94.35) (end 148.94484 94.47614) (width 0.5) (layer F.Cu) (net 1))
 (segment (start 149.1 94) (end 149.12484 94.02484) (width 0.5) (layer F.Cu) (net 1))
 (segment (start 149.12484 94.02484) (end 148.94484 94.47614) (width 0.25) (layer F.Cu) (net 1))
 (segment (start 149.13 94.48) (end 149.03 94.53) (width 0.25) (layer B.Cu) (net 1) (status 30))
 (segment (start 149.03 94.53) (end 149.08 94.48) (width 0.25) (layer B.Cu) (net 1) (status 30))
 (segment (start 149.5 95.47) (end 149.5 95) (width 0.5) (layer B.Cu) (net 1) (status 20))
 (segment (start 149.5 95) (end 149.65 94.5) (width 0.25) (layer B.Cu) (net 1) (status 20))
 (segment (start 149.65 94.5) (end 149.65 94.5) (width 0.25) (layer B.Cu) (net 1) (status 20))
 (segment (start 149.65 94.5) (end 149.23 94.58) (width 0.25) (layer B.Cu) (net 1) (status 20))
 (via (at 149.13 94.48) (size 0.6) (drill 0.4) (layers F.Cu B.Cu) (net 1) (status 30))
 (segment (start 149.23 94.58) (end 149.13 94.48) (width 0.25) (layer B.Cu) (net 1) (status 30))
 (segment (start 145.71 94.14) (end 146.3 94.15) (width 0.5) (layer F.Cu) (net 4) (status 10))
 (segment (start 146.3 94.15) (end 146.66 94.55) (width 0.5) (layer F.Cu) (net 4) (status 10))
 (segment (start 146.66 94.55) (end 146.62548 94.42614) (width 0.25) (layer F.Cu) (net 4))
 (segment (start 147.5 95.47) (end 147.5 94.97) (width 0.25) (layer B.Cu) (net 4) (status 30))
 (segment (start 147.5 94.97) (end 147.32 94.78) (width 0.25) (layer B.Cu) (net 4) (status 10))
 (segment (start 147.32 94.78) (end 146.63 94.51) (width 0.25) (layer B.Cu) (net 4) (status 10))
 (via (at 146.63 94.51) (size 0.6) (drill 0.4) (layers F.Cu B.Cu) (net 4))
 (segment (start 146.63 94.51) (end 146.65548 94.53548) (width 0.25) (layer F.Cu) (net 4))
 (segment (start 146.65548 94.53548) (end 146.62548 94.42614) (width 0.25) (layer F.Cu) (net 4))
 (segment (start 151.21 94.15) (end 150.75 94.15) (width 0.5) (layer F.Cu) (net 3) (status 10))
 (segment (start 150.75 94.15) (end 150.37452 94.77614) (width 0.5) (layer F.Cu) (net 3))
 (segment (start 150.5 95.47) (end 150.5 94.95) (width 0.25) (layer B.Cu) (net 3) (status 10))
 (segment (start 150.3 94.75) (end 150.6 94.3) (width 0.25) (layer F.Cu) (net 3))
 (via (at 150.3 94.75) (size 0.6) (drill 0.4) (layers F.Cu B.Cu) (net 3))
 (segment (start 150.5 94.95) (end 150.3 94.75) (width 0.25) (layer B.Cu) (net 3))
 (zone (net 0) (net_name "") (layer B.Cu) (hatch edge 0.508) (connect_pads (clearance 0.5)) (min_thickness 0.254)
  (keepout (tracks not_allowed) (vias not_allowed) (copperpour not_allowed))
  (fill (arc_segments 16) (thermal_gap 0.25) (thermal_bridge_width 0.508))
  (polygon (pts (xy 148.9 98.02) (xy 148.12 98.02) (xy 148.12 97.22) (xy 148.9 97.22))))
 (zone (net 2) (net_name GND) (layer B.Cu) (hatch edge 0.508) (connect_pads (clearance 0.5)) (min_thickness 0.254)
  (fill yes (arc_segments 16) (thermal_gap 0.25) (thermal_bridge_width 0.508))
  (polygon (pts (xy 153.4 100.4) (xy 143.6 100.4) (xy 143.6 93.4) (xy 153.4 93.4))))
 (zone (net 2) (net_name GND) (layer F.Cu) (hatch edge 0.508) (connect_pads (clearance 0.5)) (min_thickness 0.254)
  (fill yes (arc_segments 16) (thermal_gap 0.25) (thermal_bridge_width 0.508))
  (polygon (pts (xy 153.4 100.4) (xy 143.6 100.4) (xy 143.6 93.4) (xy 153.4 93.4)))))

